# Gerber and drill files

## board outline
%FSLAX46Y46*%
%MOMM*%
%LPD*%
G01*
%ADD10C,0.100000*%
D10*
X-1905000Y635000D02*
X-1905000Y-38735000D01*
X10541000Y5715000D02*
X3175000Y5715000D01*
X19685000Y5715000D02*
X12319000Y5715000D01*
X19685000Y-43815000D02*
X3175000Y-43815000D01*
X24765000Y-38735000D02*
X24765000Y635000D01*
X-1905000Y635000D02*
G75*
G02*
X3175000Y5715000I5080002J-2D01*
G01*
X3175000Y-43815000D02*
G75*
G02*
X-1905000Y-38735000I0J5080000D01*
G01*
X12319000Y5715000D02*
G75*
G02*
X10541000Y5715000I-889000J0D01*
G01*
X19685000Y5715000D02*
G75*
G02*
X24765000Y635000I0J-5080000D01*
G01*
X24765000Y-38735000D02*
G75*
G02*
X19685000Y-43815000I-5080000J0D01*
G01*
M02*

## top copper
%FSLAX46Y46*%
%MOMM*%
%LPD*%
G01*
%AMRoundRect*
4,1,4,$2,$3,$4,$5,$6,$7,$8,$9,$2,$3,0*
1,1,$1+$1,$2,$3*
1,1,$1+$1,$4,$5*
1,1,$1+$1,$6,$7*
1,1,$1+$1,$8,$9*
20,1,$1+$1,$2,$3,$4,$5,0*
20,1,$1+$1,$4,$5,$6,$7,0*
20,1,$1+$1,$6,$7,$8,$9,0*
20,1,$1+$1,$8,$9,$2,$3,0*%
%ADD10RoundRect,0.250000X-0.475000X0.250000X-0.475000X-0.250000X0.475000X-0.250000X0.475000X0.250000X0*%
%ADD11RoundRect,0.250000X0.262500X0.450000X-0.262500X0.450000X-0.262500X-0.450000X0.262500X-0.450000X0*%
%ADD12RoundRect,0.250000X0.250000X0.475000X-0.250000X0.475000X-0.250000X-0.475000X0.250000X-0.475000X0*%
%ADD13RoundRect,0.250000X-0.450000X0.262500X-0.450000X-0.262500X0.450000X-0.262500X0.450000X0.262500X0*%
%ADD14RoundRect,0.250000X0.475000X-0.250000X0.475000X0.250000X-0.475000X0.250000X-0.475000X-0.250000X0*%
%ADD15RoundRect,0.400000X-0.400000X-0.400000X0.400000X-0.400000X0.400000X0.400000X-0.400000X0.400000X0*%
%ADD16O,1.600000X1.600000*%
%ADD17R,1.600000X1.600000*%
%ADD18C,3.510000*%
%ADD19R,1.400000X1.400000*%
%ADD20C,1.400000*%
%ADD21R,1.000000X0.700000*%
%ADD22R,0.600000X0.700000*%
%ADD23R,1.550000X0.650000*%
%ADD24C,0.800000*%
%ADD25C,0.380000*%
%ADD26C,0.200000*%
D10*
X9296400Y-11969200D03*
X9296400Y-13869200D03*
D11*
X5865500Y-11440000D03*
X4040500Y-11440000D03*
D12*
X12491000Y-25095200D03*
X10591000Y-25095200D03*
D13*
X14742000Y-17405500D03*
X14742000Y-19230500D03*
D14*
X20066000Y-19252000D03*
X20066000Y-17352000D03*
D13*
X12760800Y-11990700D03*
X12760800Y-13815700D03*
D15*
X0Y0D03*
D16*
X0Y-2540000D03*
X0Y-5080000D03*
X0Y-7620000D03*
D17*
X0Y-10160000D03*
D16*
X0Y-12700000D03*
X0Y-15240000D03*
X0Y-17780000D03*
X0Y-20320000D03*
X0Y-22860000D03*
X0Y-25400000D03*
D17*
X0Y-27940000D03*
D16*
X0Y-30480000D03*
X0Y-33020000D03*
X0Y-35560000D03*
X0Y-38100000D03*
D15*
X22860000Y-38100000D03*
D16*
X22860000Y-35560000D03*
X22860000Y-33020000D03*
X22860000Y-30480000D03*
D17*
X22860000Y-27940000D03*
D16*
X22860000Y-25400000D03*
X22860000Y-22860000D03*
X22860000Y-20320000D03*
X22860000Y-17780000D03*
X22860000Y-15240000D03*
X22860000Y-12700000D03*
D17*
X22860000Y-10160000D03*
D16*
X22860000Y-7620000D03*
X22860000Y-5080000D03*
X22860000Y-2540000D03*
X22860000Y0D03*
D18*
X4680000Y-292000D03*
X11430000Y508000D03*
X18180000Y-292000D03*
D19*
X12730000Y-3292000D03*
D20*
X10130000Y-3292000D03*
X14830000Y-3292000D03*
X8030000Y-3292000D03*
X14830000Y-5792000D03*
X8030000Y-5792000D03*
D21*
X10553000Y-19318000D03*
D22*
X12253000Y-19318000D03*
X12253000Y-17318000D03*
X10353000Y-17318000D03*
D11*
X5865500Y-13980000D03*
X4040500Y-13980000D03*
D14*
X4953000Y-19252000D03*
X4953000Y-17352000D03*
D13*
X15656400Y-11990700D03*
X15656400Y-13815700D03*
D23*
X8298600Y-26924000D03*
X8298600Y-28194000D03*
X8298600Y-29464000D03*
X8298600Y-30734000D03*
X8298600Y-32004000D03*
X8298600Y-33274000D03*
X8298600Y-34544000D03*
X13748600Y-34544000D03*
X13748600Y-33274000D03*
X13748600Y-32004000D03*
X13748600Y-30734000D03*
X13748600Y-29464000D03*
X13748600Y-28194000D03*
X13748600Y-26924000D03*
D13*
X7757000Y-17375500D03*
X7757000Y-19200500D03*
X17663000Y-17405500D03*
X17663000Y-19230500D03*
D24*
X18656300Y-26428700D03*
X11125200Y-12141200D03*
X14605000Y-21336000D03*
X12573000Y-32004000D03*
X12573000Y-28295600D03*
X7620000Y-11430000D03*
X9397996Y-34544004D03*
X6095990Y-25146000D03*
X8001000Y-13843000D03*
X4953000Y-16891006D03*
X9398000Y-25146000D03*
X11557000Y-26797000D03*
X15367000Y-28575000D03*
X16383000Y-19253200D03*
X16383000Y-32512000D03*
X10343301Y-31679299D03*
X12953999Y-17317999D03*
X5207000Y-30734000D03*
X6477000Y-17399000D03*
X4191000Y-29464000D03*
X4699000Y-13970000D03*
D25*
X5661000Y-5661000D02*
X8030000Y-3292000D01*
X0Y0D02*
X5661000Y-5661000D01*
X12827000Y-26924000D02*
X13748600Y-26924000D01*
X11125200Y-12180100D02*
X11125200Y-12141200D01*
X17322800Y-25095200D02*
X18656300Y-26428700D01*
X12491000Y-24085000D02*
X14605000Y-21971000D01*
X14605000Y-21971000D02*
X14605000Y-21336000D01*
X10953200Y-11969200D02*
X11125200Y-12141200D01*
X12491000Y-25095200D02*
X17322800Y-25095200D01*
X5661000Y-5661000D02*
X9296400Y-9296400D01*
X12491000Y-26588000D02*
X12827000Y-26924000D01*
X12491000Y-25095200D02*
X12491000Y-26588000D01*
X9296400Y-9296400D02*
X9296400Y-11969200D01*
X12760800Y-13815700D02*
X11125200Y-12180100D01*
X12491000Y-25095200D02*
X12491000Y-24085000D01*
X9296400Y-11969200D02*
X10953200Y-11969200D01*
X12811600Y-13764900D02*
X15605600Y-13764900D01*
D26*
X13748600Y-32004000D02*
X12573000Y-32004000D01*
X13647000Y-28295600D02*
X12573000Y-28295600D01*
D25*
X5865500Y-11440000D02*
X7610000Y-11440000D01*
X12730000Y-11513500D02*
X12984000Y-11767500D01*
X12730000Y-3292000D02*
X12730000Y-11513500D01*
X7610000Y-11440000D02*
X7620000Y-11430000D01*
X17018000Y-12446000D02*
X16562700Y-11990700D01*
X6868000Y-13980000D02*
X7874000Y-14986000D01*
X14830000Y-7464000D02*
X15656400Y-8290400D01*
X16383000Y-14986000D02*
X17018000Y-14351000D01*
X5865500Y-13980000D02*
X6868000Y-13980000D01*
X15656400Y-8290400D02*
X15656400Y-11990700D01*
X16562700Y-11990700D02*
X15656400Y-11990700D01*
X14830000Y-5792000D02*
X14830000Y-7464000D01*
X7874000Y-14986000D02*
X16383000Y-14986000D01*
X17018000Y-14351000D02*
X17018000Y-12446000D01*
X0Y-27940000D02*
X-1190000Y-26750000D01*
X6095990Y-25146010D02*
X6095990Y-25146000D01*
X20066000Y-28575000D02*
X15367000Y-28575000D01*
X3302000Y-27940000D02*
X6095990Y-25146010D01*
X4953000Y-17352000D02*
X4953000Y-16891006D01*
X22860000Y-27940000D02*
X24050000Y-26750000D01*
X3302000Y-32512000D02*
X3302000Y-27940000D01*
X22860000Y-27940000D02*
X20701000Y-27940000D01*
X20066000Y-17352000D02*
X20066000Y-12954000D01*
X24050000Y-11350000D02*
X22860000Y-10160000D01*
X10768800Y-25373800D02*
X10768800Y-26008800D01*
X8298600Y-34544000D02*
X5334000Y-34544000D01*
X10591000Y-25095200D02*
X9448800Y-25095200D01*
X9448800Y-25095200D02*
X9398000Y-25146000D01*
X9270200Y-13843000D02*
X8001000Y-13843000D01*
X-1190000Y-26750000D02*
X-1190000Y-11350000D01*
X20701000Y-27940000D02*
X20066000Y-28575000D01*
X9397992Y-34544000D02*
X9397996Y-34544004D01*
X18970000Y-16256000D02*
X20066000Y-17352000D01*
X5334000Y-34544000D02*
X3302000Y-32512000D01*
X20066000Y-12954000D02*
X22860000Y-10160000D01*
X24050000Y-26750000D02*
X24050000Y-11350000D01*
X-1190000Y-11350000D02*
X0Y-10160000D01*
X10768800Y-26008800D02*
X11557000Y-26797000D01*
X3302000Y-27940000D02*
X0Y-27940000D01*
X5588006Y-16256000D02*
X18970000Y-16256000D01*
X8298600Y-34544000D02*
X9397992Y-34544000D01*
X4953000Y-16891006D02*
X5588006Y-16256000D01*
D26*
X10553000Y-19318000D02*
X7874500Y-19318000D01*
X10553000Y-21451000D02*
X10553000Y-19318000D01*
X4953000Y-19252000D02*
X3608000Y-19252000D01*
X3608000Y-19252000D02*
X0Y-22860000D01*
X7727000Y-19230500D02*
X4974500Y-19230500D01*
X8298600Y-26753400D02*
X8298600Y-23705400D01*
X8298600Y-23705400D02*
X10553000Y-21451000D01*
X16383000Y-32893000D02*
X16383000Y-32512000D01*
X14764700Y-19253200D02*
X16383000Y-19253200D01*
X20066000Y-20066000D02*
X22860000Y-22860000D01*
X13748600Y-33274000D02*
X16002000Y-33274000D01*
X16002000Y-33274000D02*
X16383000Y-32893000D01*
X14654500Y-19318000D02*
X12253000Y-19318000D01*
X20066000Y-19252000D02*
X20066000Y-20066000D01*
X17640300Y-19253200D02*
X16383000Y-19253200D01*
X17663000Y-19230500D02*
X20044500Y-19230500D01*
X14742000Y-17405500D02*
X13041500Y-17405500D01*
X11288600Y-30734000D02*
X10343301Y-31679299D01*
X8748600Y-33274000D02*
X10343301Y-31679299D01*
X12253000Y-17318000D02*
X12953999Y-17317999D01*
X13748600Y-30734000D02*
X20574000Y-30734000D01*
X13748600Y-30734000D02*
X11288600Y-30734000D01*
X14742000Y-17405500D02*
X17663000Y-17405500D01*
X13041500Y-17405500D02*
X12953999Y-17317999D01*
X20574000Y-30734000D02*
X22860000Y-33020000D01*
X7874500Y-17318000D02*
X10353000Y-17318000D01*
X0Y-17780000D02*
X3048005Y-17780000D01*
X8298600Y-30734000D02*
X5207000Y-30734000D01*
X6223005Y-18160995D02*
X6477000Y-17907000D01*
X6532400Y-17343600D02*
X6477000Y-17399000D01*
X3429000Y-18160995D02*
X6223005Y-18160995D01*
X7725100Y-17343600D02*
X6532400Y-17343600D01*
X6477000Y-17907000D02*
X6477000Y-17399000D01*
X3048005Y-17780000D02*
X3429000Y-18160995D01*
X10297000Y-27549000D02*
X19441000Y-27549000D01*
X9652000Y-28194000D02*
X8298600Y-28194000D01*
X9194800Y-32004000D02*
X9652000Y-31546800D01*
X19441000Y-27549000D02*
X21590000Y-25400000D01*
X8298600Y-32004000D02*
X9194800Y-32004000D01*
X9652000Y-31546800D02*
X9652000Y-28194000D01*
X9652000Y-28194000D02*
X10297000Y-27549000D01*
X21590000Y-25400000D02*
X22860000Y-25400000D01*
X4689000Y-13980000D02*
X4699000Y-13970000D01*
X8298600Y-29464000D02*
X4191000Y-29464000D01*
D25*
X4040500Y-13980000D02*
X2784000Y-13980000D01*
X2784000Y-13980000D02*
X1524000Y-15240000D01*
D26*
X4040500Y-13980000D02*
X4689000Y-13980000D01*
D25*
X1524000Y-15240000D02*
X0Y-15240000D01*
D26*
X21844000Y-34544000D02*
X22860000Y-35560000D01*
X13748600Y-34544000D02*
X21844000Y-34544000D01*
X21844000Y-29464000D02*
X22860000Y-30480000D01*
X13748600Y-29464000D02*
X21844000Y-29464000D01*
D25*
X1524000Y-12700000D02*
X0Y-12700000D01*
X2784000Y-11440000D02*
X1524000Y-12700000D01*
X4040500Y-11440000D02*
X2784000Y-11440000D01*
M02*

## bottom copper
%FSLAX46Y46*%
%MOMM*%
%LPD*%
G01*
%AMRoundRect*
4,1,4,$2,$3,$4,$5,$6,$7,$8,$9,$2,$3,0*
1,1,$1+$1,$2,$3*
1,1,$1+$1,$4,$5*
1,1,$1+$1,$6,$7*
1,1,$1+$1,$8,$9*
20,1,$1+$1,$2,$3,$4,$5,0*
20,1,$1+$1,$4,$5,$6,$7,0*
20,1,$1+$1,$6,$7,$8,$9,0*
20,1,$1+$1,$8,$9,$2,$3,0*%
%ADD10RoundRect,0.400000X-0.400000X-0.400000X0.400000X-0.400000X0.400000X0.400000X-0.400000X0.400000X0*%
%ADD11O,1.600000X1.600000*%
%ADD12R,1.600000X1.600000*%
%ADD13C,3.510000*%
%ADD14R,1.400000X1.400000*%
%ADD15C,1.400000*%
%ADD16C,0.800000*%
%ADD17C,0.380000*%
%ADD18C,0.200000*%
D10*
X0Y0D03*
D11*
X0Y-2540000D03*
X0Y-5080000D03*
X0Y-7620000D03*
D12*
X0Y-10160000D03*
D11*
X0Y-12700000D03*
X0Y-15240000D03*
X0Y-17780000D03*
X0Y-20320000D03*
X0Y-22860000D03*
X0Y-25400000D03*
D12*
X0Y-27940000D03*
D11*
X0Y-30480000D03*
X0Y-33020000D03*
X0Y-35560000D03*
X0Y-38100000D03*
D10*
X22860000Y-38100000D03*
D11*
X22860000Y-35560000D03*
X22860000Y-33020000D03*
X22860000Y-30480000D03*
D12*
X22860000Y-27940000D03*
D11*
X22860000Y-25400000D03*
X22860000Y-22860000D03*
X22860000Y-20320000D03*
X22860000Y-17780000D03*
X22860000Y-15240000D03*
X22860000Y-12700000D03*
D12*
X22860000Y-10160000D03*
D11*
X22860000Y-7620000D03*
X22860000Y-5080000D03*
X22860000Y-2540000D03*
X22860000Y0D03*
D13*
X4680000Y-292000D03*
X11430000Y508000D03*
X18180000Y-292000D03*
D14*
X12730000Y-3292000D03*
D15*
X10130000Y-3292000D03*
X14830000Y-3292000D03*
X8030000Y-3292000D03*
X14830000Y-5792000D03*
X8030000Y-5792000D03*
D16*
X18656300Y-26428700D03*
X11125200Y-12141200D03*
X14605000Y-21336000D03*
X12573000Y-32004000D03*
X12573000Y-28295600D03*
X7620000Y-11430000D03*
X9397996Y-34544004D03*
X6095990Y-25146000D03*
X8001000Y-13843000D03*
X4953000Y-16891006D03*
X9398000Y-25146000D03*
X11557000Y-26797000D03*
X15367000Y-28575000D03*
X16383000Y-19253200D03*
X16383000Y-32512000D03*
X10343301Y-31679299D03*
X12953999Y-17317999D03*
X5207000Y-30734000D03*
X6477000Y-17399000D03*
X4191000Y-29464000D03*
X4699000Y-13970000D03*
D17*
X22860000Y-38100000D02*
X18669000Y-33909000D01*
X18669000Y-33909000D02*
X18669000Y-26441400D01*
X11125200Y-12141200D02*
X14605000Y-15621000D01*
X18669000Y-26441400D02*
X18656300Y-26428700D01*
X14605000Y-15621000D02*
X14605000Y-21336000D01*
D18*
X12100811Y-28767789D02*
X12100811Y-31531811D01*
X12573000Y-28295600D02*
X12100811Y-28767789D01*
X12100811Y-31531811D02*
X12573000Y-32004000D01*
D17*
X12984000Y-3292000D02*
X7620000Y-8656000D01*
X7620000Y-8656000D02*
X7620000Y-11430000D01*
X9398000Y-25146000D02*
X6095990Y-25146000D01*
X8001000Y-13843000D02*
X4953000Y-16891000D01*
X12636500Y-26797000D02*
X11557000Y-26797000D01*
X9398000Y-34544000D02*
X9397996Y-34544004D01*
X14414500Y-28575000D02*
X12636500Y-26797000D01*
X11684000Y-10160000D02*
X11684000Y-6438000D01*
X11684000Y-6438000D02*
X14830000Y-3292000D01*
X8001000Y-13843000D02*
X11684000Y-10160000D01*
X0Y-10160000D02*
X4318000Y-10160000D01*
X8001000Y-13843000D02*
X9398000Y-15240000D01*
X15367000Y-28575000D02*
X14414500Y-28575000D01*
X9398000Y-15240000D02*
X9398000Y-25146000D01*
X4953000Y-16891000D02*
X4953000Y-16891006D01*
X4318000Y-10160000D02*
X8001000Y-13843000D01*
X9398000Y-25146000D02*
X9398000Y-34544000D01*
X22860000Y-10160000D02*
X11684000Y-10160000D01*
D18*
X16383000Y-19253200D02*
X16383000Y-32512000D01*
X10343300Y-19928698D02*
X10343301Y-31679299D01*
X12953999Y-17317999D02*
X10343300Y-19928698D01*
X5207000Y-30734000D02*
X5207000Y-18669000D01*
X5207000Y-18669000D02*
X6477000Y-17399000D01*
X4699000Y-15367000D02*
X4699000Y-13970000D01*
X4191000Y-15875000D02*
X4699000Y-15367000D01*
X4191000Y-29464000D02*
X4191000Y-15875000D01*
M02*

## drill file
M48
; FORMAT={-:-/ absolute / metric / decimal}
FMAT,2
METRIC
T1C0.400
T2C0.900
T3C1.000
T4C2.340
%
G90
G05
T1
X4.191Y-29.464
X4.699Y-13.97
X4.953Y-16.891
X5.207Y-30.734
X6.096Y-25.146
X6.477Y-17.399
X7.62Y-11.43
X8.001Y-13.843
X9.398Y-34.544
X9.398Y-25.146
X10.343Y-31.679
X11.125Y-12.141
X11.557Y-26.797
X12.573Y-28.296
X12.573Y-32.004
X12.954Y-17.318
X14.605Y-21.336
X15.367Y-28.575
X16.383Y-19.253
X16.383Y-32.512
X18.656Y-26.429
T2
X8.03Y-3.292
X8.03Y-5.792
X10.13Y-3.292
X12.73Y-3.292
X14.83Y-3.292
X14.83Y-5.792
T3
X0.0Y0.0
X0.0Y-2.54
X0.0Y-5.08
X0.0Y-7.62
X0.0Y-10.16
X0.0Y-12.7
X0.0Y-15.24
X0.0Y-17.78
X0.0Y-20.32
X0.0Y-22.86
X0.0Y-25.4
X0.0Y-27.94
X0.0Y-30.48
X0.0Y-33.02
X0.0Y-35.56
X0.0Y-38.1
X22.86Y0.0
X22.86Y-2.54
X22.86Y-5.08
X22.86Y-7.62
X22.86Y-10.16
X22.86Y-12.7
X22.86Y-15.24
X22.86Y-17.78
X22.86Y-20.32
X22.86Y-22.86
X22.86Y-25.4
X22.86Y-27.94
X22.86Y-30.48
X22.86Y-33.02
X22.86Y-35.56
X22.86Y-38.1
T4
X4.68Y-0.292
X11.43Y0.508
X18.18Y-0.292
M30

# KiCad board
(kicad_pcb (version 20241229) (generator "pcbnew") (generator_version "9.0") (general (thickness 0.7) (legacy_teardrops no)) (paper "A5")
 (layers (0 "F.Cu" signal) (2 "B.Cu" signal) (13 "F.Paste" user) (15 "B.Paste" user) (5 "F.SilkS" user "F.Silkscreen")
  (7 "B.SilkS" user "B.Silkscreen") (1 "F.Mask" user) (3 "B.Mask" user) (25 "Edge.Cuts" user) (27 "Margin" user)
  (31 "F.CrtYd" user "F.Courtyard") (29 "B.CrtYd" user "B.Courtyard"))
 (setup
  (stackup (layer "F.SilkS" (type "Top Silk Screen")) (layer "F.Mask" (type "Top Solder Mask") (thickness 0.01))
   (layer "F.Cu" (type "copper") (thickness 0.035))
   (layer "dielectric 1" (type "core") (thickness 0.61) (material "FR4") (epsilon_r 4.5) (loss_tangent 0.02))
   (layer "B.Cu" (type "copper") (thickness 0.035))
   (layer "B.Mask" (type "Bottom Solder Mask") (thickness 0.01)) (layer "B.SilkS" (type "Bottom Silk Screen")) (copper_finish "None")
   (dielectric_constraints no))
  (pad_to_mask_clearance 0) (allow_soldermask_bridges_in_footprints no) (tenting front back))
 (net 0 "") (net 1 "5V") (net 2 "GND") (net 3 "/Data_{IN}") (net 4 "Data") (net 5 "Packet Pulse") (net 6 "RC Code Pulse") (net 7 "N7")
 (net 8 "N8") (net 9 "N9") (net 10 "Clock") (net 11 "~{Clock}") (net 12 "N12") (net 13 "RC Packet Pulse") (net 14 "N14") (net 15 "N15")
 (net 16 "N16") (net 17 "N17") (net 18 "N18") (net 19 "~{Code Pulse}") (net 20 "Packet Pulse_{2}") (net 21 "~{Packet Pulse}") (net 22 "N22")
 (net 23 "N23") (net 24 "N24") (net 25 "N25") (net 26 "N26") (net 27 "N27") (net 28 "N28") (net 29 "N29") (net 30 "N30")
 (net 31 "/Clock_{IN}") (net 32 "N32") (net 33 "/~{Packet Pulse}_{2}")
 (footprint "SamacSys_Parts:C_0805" (layer "F.Cu") (at 9.2964 12.9032 180)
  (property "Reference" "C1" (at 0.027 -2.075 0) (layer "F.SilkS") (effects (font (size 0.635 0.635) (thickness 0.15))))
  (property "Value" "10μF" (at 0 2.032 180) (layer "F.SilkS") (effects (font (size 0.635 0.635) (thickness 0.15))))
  (pad "1" smd roundrect (at 0 0.934 270) (size 1 1.45) (layers "F.Cu" "F.Mask" "F.Paste") (roundrect_rratio 0.25) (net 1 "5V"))
  (pad "2" smd roundrect (at 0 -0.966 270) (size 1 1.45) (layers "F.Cu" "F.Mask" "F.Paste") (roundrect_rratio 0.25) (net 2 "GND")))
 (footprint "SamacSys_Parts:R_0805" (layer "F.Cu") (at 4.953 11.43 90)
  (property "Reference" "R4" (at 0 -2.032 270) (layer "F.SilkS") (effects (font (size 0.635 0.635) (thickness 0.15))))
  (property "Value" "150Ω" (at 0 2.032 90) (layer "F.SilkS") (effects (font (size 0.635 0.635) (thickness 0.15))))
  (pad "1" smd roundrect (at -0.01 0.9125 180) (size 1.025 1.4) (layers "F.Cu" "F.Mask" "F.Paste") (roundrect_rratio 0.243902)
   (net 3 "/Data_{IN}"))
  (pad "2" smd roundrect (at -0.01 -0.9125 180) (size 1.025 1.4) (layers "F.Cu" "F.Mask" "F.Paste") (roundrect_rratio 0.243902)
   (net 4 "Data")))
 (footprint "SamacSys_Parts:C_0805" (layer "F.Cu") (at 11.557 25.0952 90)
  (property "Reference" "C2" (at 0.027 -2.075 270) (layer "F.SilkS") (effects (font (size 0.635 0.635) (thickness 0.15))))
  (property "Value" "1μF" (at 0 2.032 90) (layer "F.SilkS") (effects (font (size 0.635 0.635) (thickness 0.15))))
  (pad "1" smd roundrect (at 0 0.934 180) (size 1 1.45) (layers "F.Cu" "F.Mask" "F.Paste") (roundrect_rratio 0.25) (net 1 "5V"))
  (pad "2" smd roundrect (at 0 -0.966 180) (size 1 1.45) (layers "F.Cu" "F.Mask" "F.Paste") (roundrect_rratio 0.25) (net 2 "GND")))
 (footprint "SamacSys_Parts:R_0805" (layer "F.Cu") (at 14.732 18.318 180)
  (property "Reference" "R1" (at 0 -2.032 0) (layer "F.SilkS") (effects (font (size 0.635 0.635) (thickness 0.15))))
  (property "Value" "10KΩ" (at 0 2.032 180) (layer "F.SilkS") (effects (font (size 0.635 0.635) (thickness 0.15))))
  (pad "1" smd roundrect (at -0.01 0.9125 270) (size 1.025 1.4) (layers "F.Cu" "F.Mask" "F.Paste") (roundrect_rratio 0.243902)
   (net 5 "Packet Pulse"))
  (pad "2" smd roundrect (at -0.01 -0.9125 270) (size 1.025 1.4) (layers "F.Cu" "F.Mask" "F.Paste") (roundrect_rratio 0.243902)
   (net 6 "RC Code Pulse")))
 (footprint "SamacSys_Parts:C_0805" (layer "F.Cu") (at 20.066 18.318)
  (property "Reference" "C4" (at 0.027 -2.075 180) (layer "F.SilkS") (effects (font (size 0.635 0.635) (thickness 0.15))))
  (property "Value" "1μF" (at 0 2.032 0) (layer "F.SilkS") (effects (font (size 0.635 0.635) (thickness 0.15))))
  (pad "1" smd roundrect (at 0 0.934 90) (size 1 1.45) (layers "F.Cu" "F.Mask" "F.Paste") (roundrect_rratio 0.25) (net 6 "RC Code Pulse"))
  (pad "2" smd roundrect (at 0 -0.966 90) (size 1 1.45) (layers "F.Cu" "F.Mask" "F.Paste") (roundrect_rratio 0.25) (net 2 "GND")))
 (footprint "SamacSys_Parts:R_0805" (layer "F.Cu") (at 12.7508 12.9032 180)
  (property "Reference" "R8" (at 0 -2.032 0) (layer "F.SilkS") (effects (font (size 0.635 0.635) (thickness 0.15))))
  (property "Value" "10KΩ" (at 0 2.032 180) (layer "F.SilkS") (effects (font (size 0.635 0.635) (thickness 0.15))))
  (pad "1" smd roundrect (at -0.01 0.9125 270) (size 1.025 1.4) (layers "F.Cu" "F.Mask" "F.Paste") (roundrect_rratio 0.243902)
   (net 3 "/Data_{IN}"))
  (pad "2" smd roundrect (at -0.01 -0.9125 270) (size 1.025 1.4) (layers "F.Cu" "F.Mask" "F.Paste") (roundrect_rratio 0.243902) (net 1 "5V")))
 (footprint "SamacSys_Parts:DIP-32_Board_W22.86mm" (layer "F.Cu") (at 0 0)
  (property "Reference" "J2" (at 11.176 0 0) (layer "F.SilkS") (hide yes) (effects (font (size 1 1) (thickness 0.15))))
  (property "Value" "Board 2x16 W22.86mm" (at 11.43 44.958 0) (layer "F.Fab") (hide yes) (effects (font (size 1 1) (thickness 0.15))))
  (fp_line (start -1.905 -0.635) (end -1.905 38.735) (stroke (width 0.1) (type solid)) (layer "Edge.Cuts"))
  (fp_line (start 10.541 -5.715) (end 3.175 -5.715) (stroke (width 0.1) (type solid)) (layer "Edge.Cuts"))
  (fp_line (start 19.685 -5.715) (end 12.319 -5.715) (stroke (width 0.1) (type solid)) (layer "Edge.Cuts"))
  (fp_line (start 19.685 43.815) (end 3.175 43.815) (stroke (width 0.1) (type solid)) (layer "Edge.Cuts"))
  (fp_line (start 24.765 38.735) (end 24.765 -0.635) (stroke (width 0.1) (type solid)) (layer "Edge.Cuts"))
  (fp_arc (start -1.905 -0.635) (mid -0.417102 -4.227102) (end 3.175 -5.715) (stroke (width 0.1) (type solid)) (layer "Edge.Cuts"))
  (fp_arc (start 3.175 43.815) (mid -0.417102 42.327102) (end -1.905 38.735) (stroke (width 0.1) (type solid)) (layer "Edge.Cuts"))
  (fp_arc (start 12.319 -5.715) (mid 11.43 -4.826) (end 10.541 -5.715) (stroke (width 0.1) (type default)) (layer "Edge.Cuts"))
  (fp_arc (start 19.685 -5.715) (mid 23.277102 -4.227102) (end 24.765 -0.635) (stroke (width 0.1) (type solid)) (layer "Edge.Cuts"))
  (fp_arc (start 24.765 38.735) (mid 23.277103 42.327103) (end 19.685 43.815) (stroke (width 0.1) (type solid)) (layer "Edge.Cuts"))
  (pad "1" thru_hole roundrect (at 0 0) (size 1.6 1.6) (drill 1) (layers "*.Cu" "*.Mask") (remove_unused_layers no) (roundrect_rratio 0.25)
   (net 1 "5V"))
  (pad "2" thru_hole oval (at 0 2.54) (size 1.6 1.6) (drill 1) (layers "*.Cu" "*.Mask") (remove_unused_layers no) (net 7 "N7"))
  (pad "3" thru_hole oval (at 0 5.08) (size 1.6 1.6) (drill 1) (layers "*.Cu" "*.Mask") (remove_unused_layers no) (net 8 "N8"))
  (pad "4" thru_hole oval (at 0 7.62) (size 1.6 1.6) (drill 1) (layers "*.Cu" "*.Mask") (remove_unused_layers no) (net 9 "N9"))
  (pad "5" thru_hole rect (at 0 10.16) (size 1.6 1.6) (drill 1) (layers "*.Cu" "*.Mask") (remove_unused_layers no) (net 2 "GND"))
  (pad "6" thru_hole oval (at 0 12.7) (size 1.6 1.6) (drill 1) (layers "*.Cu" "*.Mask") (remove_unused_layers no) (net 4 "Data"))
  (pad "7" thru_hole oval (at 0 15.24) (size 1.6 1.6) (drill 1) (layers "*.Cu" "*.Mask") (remove_unused_layers no) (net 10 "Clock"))
  (pad "8" thru_hole oval (at 0 17.78) (size 1.6 1.6) (drill 1) (layers "*.Cu" "*.Mask") (remove_unused_layers no) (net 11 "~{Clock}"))
  (pad "9" thru_hole oval (at 0 20.32) (size 1.6 1.6) (drill 1) (layers "*.Cu" "*.Mask") (remove_unused_layers no) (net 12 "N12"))
  (pad "10" thru_hole oval (at 0 22.86) (size 1.6 1.6) (drill 1) (layers "*.Cu" "*.Mask") (remove_unused_layers no)
   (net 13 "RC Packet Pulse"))
  (pad "11" thru_hole oval (at 0 25.4) (size 1.6 1.6) (drill 1) (layers "*.Cu" "*.Mask") (remove_unused_layers no) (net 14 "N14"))
  (pad "12" thru_hole rect (at 0 27.94) (size 1.6 1.6) (drill 1) (layers "*.Cu" "*.Mask") (remove_unused_layers no) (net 2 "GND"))
  (pad "13" thru_hole oval (at 0 30.48) (size 1.6 1.6) (drill 1) (layers "*.Cu" "*.Mask") (remove_unused_layers no) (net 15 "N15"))
  (pad "14" thru_hole oval (at 0 33.02) (size 1.6 1.6) (drill 1) (layers "*.Cu" "*.Mask") (remove_unused_layers no) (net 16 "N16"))
  (pad "15" thru_hole oval (at 0 35.56) (size 1.6 1.6) (drill 1) (layers "*.Cu" "*.Mask") (remove_unused_layers no) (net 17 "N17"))
  (pad "16" thru_hole oval (at 0 38.1) (size 1.6 1.6) (drill 1) (layers "*.Cu" "*.Mask") (remove_unused_layers no) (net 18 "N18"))
  (pad "17" thru_hole roundrect (at 22.86 38.1) (size 1.6 1.6) (drill 1) (layers "*.Cu" "*.Mask") (remove_unused_layers no)
   (roundrect_rratio 0.25) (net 1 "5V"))
  (pad "18" thru_hole oval (at 22.86 35.56) (size 1.6 1.6) (drill 1) (layers "*.Cu" "*.Mask") (remove_unused_layers no)
   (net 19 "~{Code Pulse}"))
  (pad "19" thru_hole oval (at 22.86 33.02) (size 1.6 1.6) (drill 1) (layers "*.Cu" "*.Mask") (remove_unused_layers no)
   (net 5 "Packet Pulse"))
  (pad "20" thru_hole oval (at 22.86 30.48) (size 1.6 1.6) (drill 1) (layers "*.Cu" "*.Mask") (remove_unused_layers no)
   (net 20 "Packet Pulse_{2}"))
  (pad "21" thru_hole rect (at 22.86 27.94) (size 1.6 1.6) (drill 1) (layers "*.Cu" "*.Mask") (remove_unused_layers no) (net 2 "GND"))
  (pad "22" thru_hole oval (at 22.86 25.4) (size 1.6 1.6) (drill 1) (layers "*.Cu" "*.Mask") (remove_unused_layers no)
   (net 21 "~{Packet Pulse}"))
  (pad "23" thru_hole oval (at 22.86 22.86) (size 1.6 1.6) (drill 1) (layers "*.Cu" "*.Mask") (remove_unused_layers no)
   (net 6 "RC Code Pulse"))
  (pad "24" thru_hole oval (at 22.86 20.32) (size 1.6 1.6) (drill 1) (layers "*.Cu" "*.Mask") (remove_unused_layers no) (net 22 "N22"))
  (pad "25" thru_hole oval (at 22.86 17.78) (size 1.6 1.6) (drill 1) (layers "*.Cu" "*.Mask") (remove_unused_layers no) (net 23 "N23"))
  (pad "26" thru_hole oval (at 22.86 15.24) (size 1.6 1.6) (drill 1) (layers "*.Cu" "*.Mask") (remove_unused_layers no) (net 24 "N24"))
  (pad "27" thru_hole oval (at 22.86 12.7) (size 1.6 1.6) (drill 1) (layers "*.Cu" "*.Mask") (remove_unused_layers no) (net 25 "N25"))
  (pad "28" thru_hole rect (at 22.86 10.16) (size 1.6 1.6) (drill 1) (layers "*.Cu" "*.Mask") (remove_unused_layers no) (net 2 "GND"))
  (pad "29" thru_hole oval (at 22.86 7.62) (size 1.6 1.6) (drill 1) (layers "*.Cu" "*.Mask") (remove_unused_layers no) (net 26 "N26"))
  (pad "30" thru_hole oval (at 22.86 5.08) (size 1.6 1.6) (drill 1) (layers "*.Cu" "*.Mask") (remove_unused_layers no) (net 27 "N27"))
  (pad "31" thru_hole oval (at 22.86 2.54) (size 1.6 1.6) (drill 1) (layers "*.Cu" "*.Mask") (remove_unused_layers no) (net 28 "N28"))
  (pad "32" thru_hole oval (at 22.86 0) (size 1.6 1.6) (drill 1) (layers "*.Cu" "*.Mask") (remove_unused_layers no) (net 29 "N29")))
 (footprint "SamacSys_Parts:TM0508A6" (layer "F.Cu") (at 12.73 3.292)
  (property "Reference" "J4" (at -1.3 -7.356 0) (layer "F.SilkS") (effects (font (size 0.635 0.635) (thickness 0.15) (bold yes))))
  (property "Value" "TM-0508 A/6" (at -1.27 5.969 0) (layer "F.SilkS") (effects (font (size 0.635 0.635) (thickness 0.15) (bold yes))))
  (pad "" thru_hole circle (at -8.05 -3) (size 3.51 3.51) (drill 2.34) (layers "*.Cu" "*.Mask") (remove_unused_layers no))
  (pad "" thru_hole circle (at -1.3 -3.8) (size 3.51 3.51) (drill 2.34) (layers "*.Cu" "*.Mask") (remove_unused_layers no))
  (pad "" thru_hole circle (at 5.45 -3) (size 3.51 3.51) (drill 2.34) (layers "*.Cu" "*.Mask") (remove_unused_layers no))
  (pad "1" thru_hole rect (at 0 0) (size 1.4 1.4) (drill 0.9) (layers "*.Cu" "*.Mask") (remove_unused_layers no) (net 3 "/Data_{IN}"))
  (pad "2" thru_hole circle (at -2.6 0) (size 1.4 1.4) (drill 0.9) (layers "*.Cu" "*.Mask") (remove_unused_layers no) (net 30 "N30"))
  (pad "3" thru_hole circle (at 2.1 0) (size 1.4 1.4) (drill 0.9) (layers "*.Cu" "*.Mask") (remove_unused_layers no) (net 2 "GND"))
  (pad "4" thru_hole circle (at -4.7 0) (size 1.4 1.4) (drill 0.9) (layers "*.Cu" "*.Mask") (remove_unused_layers no) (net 1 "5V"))
  (pad "5" thru_hole circle (at 2.1 2.5) (size 1.4 1.4) (drill 0.9) (layers "*.Cu" "*.Mask") (remove_unused_layers no)
   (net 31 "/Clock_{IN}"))
  (pad "6" thru_hole circle (at -4.7 2.5) (size 1.4 1.4) (drill 0.9) (layers "*.Cu" "*.Mask") (remove_unused_layers no) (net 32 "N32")))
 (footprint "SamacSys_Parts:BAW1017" (layer "F.Cu") (at 11.303 18.318)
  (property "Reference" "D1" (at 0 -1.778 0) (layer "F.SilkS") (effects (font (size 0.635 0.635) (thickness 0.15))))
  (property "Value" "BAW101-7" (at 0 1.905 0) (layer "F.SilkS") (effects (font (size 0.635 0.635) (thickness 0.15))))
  (pad "1" smd rect (at -0.75 1 90) (size 0.7 1) (layers "F.Cu" "F.Mask" "F.Paste") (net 13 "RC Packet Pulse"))
  (pad "2" smd rect (at 0.95 1) (size 0.6 0.7) (layers "F.Cu" "F.Mask" "F.Paste") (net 6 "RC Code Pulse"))
  (pad "3" smd rect (at 0.95 -1) (size 0.6 0.7) (layers "F.Cu" "F.Mask" "F.Paste") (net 5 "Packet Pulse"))
  (pad "4" smd rect (at -0.95 -1) (size 0.6 0.7) (layers "F.Cu" "F.Mask" "F.Paste") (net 11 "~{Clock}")))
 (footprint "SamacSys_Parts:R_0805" (layer "F.Cu") (at 4.953 13.97 90)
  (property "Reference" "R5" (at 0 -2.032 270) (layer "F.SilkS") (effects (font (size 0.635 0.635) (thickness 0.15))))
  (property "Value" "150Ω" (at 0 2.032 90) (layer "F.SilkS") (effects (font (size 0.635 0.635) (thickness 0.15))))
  (pad "1" smd roundrect (at -0.01 0.9125 180) (size 1.025 1.4) (layers "F.Cu" "F.Mask" "F.Paste") (roundrect_rratio 0.243902)
   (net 31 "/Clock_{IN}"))
  (pad "2" smd roundrect (at -0.01 -0.9125 180) (size 1.025 1.4) (layers "F.Cu" "F.Mask" "F.Paste") (roundrect_rratio 0.243902)
   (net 10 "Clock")))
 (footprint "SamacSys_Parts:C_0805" (layer "F.Cu") (at 4.953 18.318)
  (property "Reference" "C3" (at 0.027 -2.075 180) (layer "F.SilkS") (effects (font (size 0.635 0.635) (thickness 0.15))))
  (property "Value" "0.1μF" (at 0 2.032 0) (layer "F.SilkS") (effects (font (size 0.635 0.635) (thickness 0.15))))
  (pad "1" smd roundrect (at 0 0.934 90) (size 1 1.45) (layers "F.Cu" "F.Mask" "F.Paste") (roundrect_rratio 0.25) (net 13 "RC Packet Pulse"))
  (pad "2" smd roundrect (at 0 -0.966 90) (size 1 1.45) (layers "F.Cu" "F.Mask" "F.Paste") (roundrect_rratio 0.25) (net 2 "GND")))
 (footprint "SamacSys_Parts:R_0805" (layer "F.Cu") (at 15.6464 12.9032 180)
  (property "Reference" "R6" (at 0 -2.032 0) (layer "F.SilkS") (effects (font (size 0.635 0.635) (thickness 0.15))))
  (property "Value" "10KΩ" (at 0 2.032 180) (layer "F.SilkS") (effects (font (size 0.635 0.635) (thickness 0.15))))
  (pad "1" smd roundrect (at -0.01 0.9125 270) (size 1.025 1.4) (layers "F.Cu" "F.Mask" "F.Paste") (roundrect_rratio 0.243902)
   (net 31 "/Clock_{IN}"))
  (pad "2" smd roundrect (at -0.01 -0.9125 270) (size 1.025 1.4) (layers "F.Cu" "F.Mask" "F.Paste") (roundrect_rratio 0.243902) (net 1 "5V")))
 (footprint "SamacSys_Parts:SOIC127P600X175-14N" (layer "F.Cu") (at 11.0236 30.734)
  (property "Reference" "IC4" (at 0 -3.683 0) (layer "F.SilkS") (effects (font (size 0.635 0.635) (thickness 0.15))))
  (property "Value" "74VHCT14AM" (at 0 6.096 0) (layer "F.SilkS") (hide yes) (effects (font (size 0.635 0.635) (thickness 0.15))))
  (pad "1" smd rect (at -2.725 -3.81 90) (size 0.65 1.55) (layers "F.Cu" "F.Mask" "F.Paste") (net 13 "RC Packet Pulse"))
  (pad "2" smd rect (at -2.725 -2.54 90) (size 0.65 1.55) (layers "F.Cu" "F.Mask" "F.Paste") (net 21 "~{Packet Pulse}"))
  (pad "3" smd rect (at -2.725 -1.27 90) (size 0.65 1.55) (layers "F.Cu" "F.Mask" "F.Paste") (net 10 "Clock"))
  (pad "4" smd rect (at -2.725 0 90) (size 0.65 1.55) (layers "F.Cu" "F.Mask" "F.Paste") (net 11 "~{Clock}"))
  (pad "5" smd rect (at -2.725 1.27 90) (size 0.65 1.55) (layers "F.Cu" "F.Mask" "F.Paste") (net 21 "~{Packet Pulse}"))
  (pad "6" smd rect (at -2.725 2.54 90) (size 0.65 1.55) (layers "F.Cu" "F.Mask" "F.Paste") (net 5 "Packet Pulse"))
  (pad "7" smd rect (at -2.725 3.81 90) (size 0.65 1.55) (layers "F.Cu" "F.Mask" "F.Paste") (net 2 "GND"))
  (pad "8" smd rect (at 2.725 3.81 90) (size 0.65 1.55) (layers "F.Cu" "F.Mask" "F.Paste") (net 19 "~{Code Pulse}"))
  (pad "9" smd rect (at 2.725 2.54 90) (size 0.65 1.55) (layers "F.Cu" "F.Mask" "F.Paste") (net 6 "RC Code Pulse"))
  (pad "10" smd rect (at 2.725 1.27 90) (size 0.65 1.55) (layers "F.Cu" "F.Mask" "F.Paste") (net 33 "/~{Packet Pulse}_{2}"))
  (pad "11" smd rect (at 2.725 0 90) (size 0.65 1.55) (layers "F.Cu" "F.Mask" "F.Paste") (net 5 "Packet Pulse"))
  (pad "12" smd rect (at 2.725 -1.27 90) (size 0.65 1.55) (layers "F.Cu" "F.Mask" "F.Paste") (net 20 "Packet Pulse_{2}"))
  (pad "13" smd rect (at 2.725 -2.54 90) (size 0.65 1.55) (layers "F.Cu" "F.Mask" "F.Paste") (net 33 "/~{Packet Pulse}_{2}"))
  (pad "14" smd rect (at 2.725 -3.81 90) (size 0.65 1.55) (layers "F.Cu" "F.Mask" "F.Paste") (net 1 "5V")))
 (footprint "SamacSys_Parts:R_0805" (layer "F.Cu") (at 7.747 18.288 180)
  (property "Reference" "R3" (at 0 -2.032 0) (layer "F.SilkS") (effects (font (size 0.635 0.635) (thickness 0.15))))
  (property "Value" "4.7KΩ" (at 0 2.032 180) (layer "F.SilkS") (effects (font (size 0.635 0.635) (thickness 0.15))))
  (pad "1" smd roundrect (at -0.01 0.9125 270) (size 1.025 1.4) (layers "F.Cu" "F.Mask" "F.Paste") (roundrect_rratio 0.243902)
   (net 11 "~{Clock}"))
  (pad "2" smd roundrect (at -0.01 -0.9125 270) (size 1.025 1.4) (layers "F.Cu" "F.Mask" "F.Paste") (roundrect_rratio 0.243902)
   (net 13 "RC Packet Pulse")))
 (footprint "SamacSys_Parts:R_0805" (layer "F.Cu") (at 17.653 18.318 180)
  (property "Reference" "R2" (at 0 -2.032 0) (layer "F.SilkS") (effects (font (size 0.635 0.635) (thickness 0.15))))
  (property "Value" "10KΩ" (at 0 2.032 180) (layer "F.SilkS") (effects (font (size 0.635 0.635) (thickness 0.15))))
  (pad "1" smd roundrect (at -0.01 0.9125 270) (size 1.025 1.4) (layers "F.Cu" "F.Mask" "F.Paste") (roundrect_rratio 0.243902)
   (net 5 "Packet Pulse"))
  (pad "2" smd roundrect (at -0.01 -0.9125 270) (size 1.025 1.4) (layers "F.Cu" "F.Mask" "F.Paste") (roundrect_rratio 0.243902)
   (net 6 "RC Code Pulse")))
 (segment (start 5.661 5.661) (end 8.03 3.292) (width 0.38) (layer "F.Cu") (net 1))
 (segment (start 0 0) (end 5.661 5.661) (width 0.38) (layer "F.Cu") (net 1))
 (segment (start 12.827 26.924) (end 13.7486 26.924) (width 0.38) (layer "F.Cu") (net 1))
 (segment (start 11.1252 12.1801) (end 11.1252 12.1412) (width 0.38) (layer "F.Cu") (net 1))
 (segment (start 17.3228 25.0952) (end 18.6563 26.4287) (width 0.38) (layer "F.Cu") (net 1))
 (segment (start 12.491 24.085) (end 14.605 21.971) (width 0.38) (layer "F.Cu") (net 1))
 (segment (start 14.605 21.971) (end 14.605 21.336) (width 0.38) (layer "F.Cu") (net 1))
 (segment (start 10.9532 11.9692) (end 11.1252 12.1412) (width 0.38) (layer "F.Cu") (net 1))
 (segment (start 12.491 25.0952) (end 17.3228 25.0952) (width 0.38) (layer "F.Cu") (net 1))
 (segment (start 5.661 5.661) (end 9.2964 9.2964) (width 0.38) (layer "F.Cu") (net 1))
 (segment (start 12.491 26.588) (end 12.827 26.924) (width 0.38) (layer "F.Cu") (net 1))
 (segment (start 12.491 25.0952) (end 12.491 26.588) (width 0.38) (layer "F.Cu") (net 1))
 (segment (start 9.2964 9.2964) (end 9.2964 11.9692) (width 0.38) (layer "F.Cu") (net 1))
 (segment (start 12.7608 13.8157) (end 11.1252 12.1801) (width 0.38) (layer "F.Cu") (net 1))
 (segment (start 12.491 25.0952) (end 12.491 24.085) (width 0.38) (layer "F.Cu") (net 1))
 (segment (start 9.2964 11.9692) (end 10.9532 11.9692) (width 0.38) (layer "F.Cu") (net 1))
 (segment (start 12.8116 13.7649) (end 15.6056 13.7649) (width 0.38) (layer "F.Cu") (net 1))
 (via (at 18.6563 26.4287) (size 0.8) (drill 0.4) (layers "F.Cu" "B.Cu") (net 1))
 (via (at 11.1252 12.1412) (size 0.8) (drill 0.4) (layers "F.Cu" "B.Cu") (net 1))
 (via (at 14.605 21.336) (size 0.8) (drill 0.4) (layers "F.Cu" "B.Cu") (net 1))
 (segment (start 22.86 38.1) (end 18.669 33.909) (width 0.38) (layer "B.Cu") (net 1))
 (segment (start 18.669 33.909) (end 18.669 26.4414) (width 0.38) (layer "B.Cu") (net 1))
 (segment (start 11.1252 12.1412) (end 14.605 15.621) (width 0.38) (layer "B.Cu") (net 1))
 (segment (start 18.669 26.4414) (end 18.6563 26.4287) (width 0.38) (layer "B.Cu") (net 1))
 (segment (start 14.605 15.621) (end 14.605 21.336) (width 0.38) (layer "B.Cu") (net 1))
 (segment (start 13.7486 32.004) (end 12.573 32.004) (width 0.2) (layer "F.Cu") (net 33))
 (segment (start 13.647 28.2956) (end 12.573 28.2956) (width 0.2) (layer "F.Cu") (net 33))
 (via (at 12.573 32.004) (size 0.8) (drill 0.4) (layers "F.Cu" "B.Cu") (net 33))
 (via (at 12.573 28.2956) (size 0.8) (drill 0.4) (layers "F.Cu" "B.Cu") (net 33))
 (segment (start 12.100811 28.767789) (end 12.100811 31.531811) (width 0.2) (layer "B.Cu") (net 33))
 (segment (start 12.573 28.2956) (end 12.100811 28.767789) (width 0.2) (layer "B.Cu") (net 33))
 (segment (start 12.100811 31.531811) (end 12.573 32.004) (width 0.2) (layer "B.Cu") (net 33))
 (segment (start 5.8655 11.44) (end 7.61 11.44) (width 0.38) (layer "F.Cu") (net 3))
 (segment (start 12.73 11.5135) (end 12.984 11.7675) (width 0.38) (layer "F.Cu") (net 3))
 (segment (start 12.73 3.292) (end 12.73 11.5135) (width 0.38) (layer "F.Cu") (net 3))
 (segment (start 7.61 11.44) (end 7.62 11.43) (width 0.38) (layer "F.Cu") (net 3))
 (via (at 7.62 11.43) (size 0.8) (drill 0.4) (layers "F.Cu" "B.Cu") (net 3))
 (segment (start 12.984 3.292) (end 7.62 8.656) (width 0.38) (layer "B.Cu") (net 3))
 (segment (start 7.62 8.656) (end 7.62 11.43) (width 0.38) (layer "B.Cu") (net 3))
 (segment (start 17.018 12.446) (end 16.5627 11.9907) (width 0.38) (layer "F.Cu") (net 31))
 (segment (start 6.868 13.98) (end 7.874 14.986) (width 0.38) (layer "F.Cu") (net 31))
 (segment (start 14.83 7.464) (end 15.6564 8.2904) (width 0.38) (layer "F.Cu") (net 31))
 (segment (start 16.383 14.986) (end 17.018 14.351) (width 0.38) (layer "F.Cu") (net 31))
 (segment (start 5.8655 13.98) (end 6.868 13.98) (width 0.38) (layer "F.Cu") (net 31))
 (segment (start 15.6564 8.2904) (end 15.6564 11.9907) (width 0.38) (layer "F.Cu") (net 31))
 (segment (start 16.5627 11.9907) (end 15.6564 11.9907) (width 0.38) (layer "F.Cu") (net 31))
 (segment (start 14.83 5.792) (end 14.83 7.464) (width 0.38) (layer "F.Cu") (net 31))
 (segment (start 7.874 14.986) (end 16.383 14.986) (width 0.38) (layer "F.Cu") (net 31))
 (segment (start 17.018 14.351) (end 17.018 12.446) (width 0.38) (layer "F.Cu") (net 31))
 (segment (start 0 27.94) (end -1.19 26.75) (width 0.38) (layer "F.Cu") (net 2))
 (segment (start 6.09599 25.14601) (end 6.09599 25.146) (width 0.38) (layer "F.Cu") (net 2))
 (segment (start 20.066 28.575) (end 15.367 28.575) (width 0.38) (layer "F.Cu") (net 2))
 (segment (start 3.302 27.94) (end 6.09599 25.14601) (width 0.38) (layer "F.Cu") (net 2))
 (segment (start 4.953 17.352) (end 4.953 16.891006) (width 0.38) (layer "F.Cu") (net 2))
 (segment (start 22.86 27.94) (end 24.05 26.75) (width 0.38) (layer "F.Cu") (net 2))
 (segment (start 3.302 32.512) (end 3.302 27.94) (width 0.38) (layer "F.Cu") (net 2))
 (segment (start 22.86 27.94) (end 20.701 27.94) (width 0.38) (layer "F.Cu") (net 2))
 (segment (start 20.066 17.352) (end 20.066 12.954) (width 0.38) (layer "F.Cu") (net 2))
 (segment (start 24.05 11.35) (end 22.86 10.16) (width 0.38) (layer "F.Cu") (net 2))
 (segment (start 10.7688 25.3738) (end 10.7688 26.0088) (width 0.38) (layer "F.Cu") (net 2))
 (segment (start 8.2986 34.544) (end 5.334 34.544) (width 0.38) (layer "F.Cu") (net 2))
 (segment (start 10.591 25.0952) (end 9.4488 25.0952) (width 0.38) (layer "F.Cu") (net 2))
 (segment (start 9.4488 25.0952) (end 9.398 25.146) (width 0.38) (layer "F.Cu") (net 2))
 (segment (start 9.2702 13.843) (end 8.001 13.843) (width 0.38) (layer "F.Cu") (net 2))
 (segment (start -1.19 26.75) (end -1.19 11.35) (width 0.38) (layer "F.Cu") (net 2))
 (segment (start 20.701 27.94) (end 20.066 28.575) (width 0.38) (layer "F.Cu") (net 2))
 (segment (start 9.397992 34.544) (end 9.397996 34.544004) (width 0.38) (layer "F.Cu") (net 2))
 (segment (start 18.97 16.256) (end 20.066 17.352) (width 0.38) (layer "F.Cu") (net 2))
 (segment (start 5.334 34.544) (end 3.302 32.512) (width 0.38) (layer "F.Cu") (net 2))
 (segment (start 20.066 12.954) (end 22.86 10.16) (width 0.38) (layer "F.Cu") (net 2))
 (segment (start 24.05 26.75) (end 24.05 11.35) (width 0.38) (layer "F.Cu") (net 2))
 (segment (start -1.19 11.35) (end 0 10.16) (width 0.38) (layer "F.Cu") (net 2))
 (segment (start 10.7688 26.0088) (end 11.557 26.797) (width 0.38) (layer "F.Cu") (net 2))
 (segment (start 3.302 27.94) (end 0 27.94) (width 0.38) (layer "F.Cu") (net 2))
 (segment (start 5.588006 16.256) (end 18.97 16.256) (width 0.38) (layer "F.Cu") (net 2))
 (segment (start 8.2986 34.544) (end 9.397992 34.544) (width 0.38) (layer "F.Cu") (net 2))
 (segment (start 4.953 16.891006) (end 5.588006 16.256) (width 0.38) (layer "F.Cu") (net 2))
 (via (at 9.397996 34.544004) (size 0.8) (drill 0.4) (layers "F.Cu" "B.Cu") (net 2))
 (via (at 6.09599 25.146) (size 0.8) (drill 0.4) (layers "F.Cu" "B.Cu") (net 2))
 (via (at 8.001 13.843) (size 0.8) (drill 0.4) (layers "F.Cu" "B.Cu") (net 2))
 (via (at 4.953 16.891006) (size 0.8) (drill 0.4) (layers "F.Cu" "B.Cu") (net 2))
 (via (at 9.398 25.146) (size 0.8) (drill 0.4) (layers "F.Cu" "B.Cu") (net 2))
 (via (at 11.557 26.797) (size 0.8) (drill 0.4) (layers "F.Cu" "B.Cu") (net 2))
 (via (at 15.367 28.575) (size 0.8) (drill 0.4) (layers "F.Cu" "B.Cu") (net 2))
 (segment (start 9.398 25.146) (end 6.09599 25.146) (width 0.38) (layer "B.Cu") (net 2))
 (segment (start 8.001 13.843) (end 4.953 16.891) (width 0.38) (layer "B.Cu") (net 2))
 (segment (start 12.6365 26.797) (end 11.557 26.797) (width 0.38) (layer "B.Cu") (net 2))
 (segment (start 9.398 34.544) (end 9.397996 34.544004) (width 0.38) (layer "B.Cu") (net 2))
 (segment (start 14.4145 28.575) (end 12.6365 26.797) (width 0.38) (layer "B.Cu") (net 2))
 (segment (start 11.684 10.16) (end 11.684 6.438) (width 0.38) (layer "B.Cu") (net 2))
 (segment (start 11.684 6.438) (end 14.83 3.292) (width 0.38) (layer "B.Cu") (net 2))
 (segment (start 8.001 13.843) (end 11.684 10.16) (width 0.38) (layer "B.Cu") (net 2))
 (segment (start 0 10.16) (end 4.318 10.16) (width 0.38) (layer "B.Cu") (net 2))
 (segment (start 8.001 13.843) (end 9.398 15.24) (width 0.38) (layer "B.Cu") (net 2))
 (segment (start 15.367 28.575) (end 14.4145 28.575) (width 0.38) (layer "B.Cu") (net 2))
 (segment (start 9.398 15.24) (end 9.398 25.146) (width 0.38) (layer "B.Cu") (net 2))
 (segment (start 4.953 16.891) (end 4.953 16.891006) (width 0.38) (layer "B.Cu") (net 2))
 (segment (start 4.318 10.16) (end 8.001 13.843) (width 0.38) (layer "B.Cu") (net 2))
 (segment (start 9.398 25.146) (end 9.398 34.544) (width 0.38) (layer "B.Cu") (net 2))
 (segment (start 22.86 10.16) (end 11.684 10.16) (width 0.38) (layer "B.Cu") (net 2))
 (segment (start 10.553 19.318) (end 7.8745 19.318) (width 0.2) (layer "F.Cu") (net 13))
 (segment (start 10.553 21.451) (end 10.553 19.318) (width 0.2) (layer "F.Cu") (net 13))
 (segment (start 4.953 19.252) (end 3.608 19.252) (width 0.2) (layer "F.Cu") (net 13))
 (segment (start 3.608 19.252) (end 0 22.86) (width 0.2) (layer "F.Cu") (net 13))
 (segment (start 7.727 19.2305) (end 4.9745 19.2305) (width 0.2) (layer "F.Cu") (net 13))
 (segment (start 8.2986 26.7534) (end 8.2986 23.7054) (width 0.2) (layer "F.Cu") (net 13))
 (segment (start 8.2986 23.7054) (end 10.553 21.451) (width 0.2) (layer "F.Cu") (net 13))
 (segment (start 16.383 32.893) (end 16.383 32.512) (width 0.2) (layer "F.Cu") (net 6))
 (segment (start 14.7647 19.2532) (end 16.383 19.2532) (width 0.2) (layer "F.Cu") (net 6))
 (segment (start 20.066 20.066) (end 22.86 22.86) (width 0.2) (layer "F.Cu") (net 6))
 (segment (start 13.7486 33.274) (end 16.002 33.274) (width 0.2) (layer "F.Cu") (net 6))
 (segment (start 16.002 33.274) (end 16.383 32.893) (width 0.2) (layer "F.Cu") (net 6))
 (segment (start 14.6545 19.318) (end 12.253 19.318) (width 0.2) (layer "F.Cu") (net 6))
 (segment (start 20.066 19.252) (end 20.066 20.066) (width 0.2) (layer "F.Cu") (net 6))
 (segment (start 17.6403 19.2532) (end 16.383 19.2532) (width 0.2) (layer "F.Cu") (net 6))
 (segment (start 17.663 19.2305) (end 20.0445 19.2305) (width 0.2) (layer "F.Cu") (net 6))
 (via (at 16.383 19.2532) (size 0.8) (drill 0.4) (layers "F.Cu" "B.Cu") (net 6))
 (via (at 16.383 32.512) (size 0.8) (drill 0.4) (layers "F.Cu" "B.Cu") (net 6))
 (segment (start 16.383 19.2532) (end 16.383 32.512) (width 0.2) (layer "B.Cu") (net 6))
 (segment (start 14.742 17.4055) (end 13.0415 17.4055) (width 0.2) (layer "F.Cu") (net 5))
 (segment (start 11.2886 30.734) (end 10.343301 31.679299) (width 0.2) (layer "F.Cu") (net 5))
 (segment (start 8.7486 33.274) (end 10.343301 31.679299) (width 0.2) (layer "F.Cu") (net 5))
 (segment (start 12.253 17.318) (end 12.953999 17.317999) (width 0.2) (layer "F.Cu") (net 5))
 (segment (start 13.7486 30.734) (end 20.574 30.734) (width 0.2) (layer "F.Cu") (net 5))
 (segment (start 13.7486 30.734) (end 11.2886 30.734) (width 0.2) (layer "F.Cu") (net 5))
 (segment (start 14.742 17.4055) (end 17.663 17.4055) (width 0.2) (layer "F.Cu") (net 5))
 (segment (start 13.0415 17.4055) (end 12.953999 17.317999) (width 0.2) (layer "F.Cu") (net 5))
 (segment (start 20.574 30.734) (end 22.86 33.02) (width 0.2) (layer "F.Cu") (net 5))
 (via (at 10.343301 31.679299) (size 0.8) (drill 0.4) (layers "F.Cu" "B.Cu") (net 5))
 (via (at 12.953999 17.317999) (size 0.8) (drill 0.4) (layers "F.Cu" "B.Cu") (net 5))
 (segment (start 10.3433 19.928698) (end 10.343301 31.679299) (width 0.2) (layer "B.Cu") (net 5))
 (segment (start 12.953999 17.317999) (end 10.3433 19.928698) (width 0.2) (layer "B.Cu") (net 5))
 (segment (start 7.8745 17.318) (end 10.353 17.318) (width 0.2) (layer "F.Cu") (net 11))
 (segment (start 0 17.78) (end 3.048005 17.78) (width 0.2) (layer "F.Cu") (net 11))
 (segment (start 8.2986 30.734) (end 5.207 30.734) (width 0.2) (layer "F.Cu") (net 11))
 (segment (start 6.223005 18.160995) (end 6.477 17.907) (width 0.2) (layer "F.Cu") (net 11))
 (segment (start 6.5324 17.3436) (end 6.477 17.399) (width 0.2) (layer "F.Cu") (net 11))
 (segment (start 3.429 18.160995) (end 6.223005 18.160995) (width 0.2) (layer "F.Cu") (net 11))
 (segment (start 7.7251 17.3436) (end 6.5324 17.3436) (width 0.2) (layer "F.Cu") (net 11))
 (segment (start 6.477 17.907) (end 6.477 17.399) (width 0.2) (layer "F.Cu") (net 11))
 (segment (start 3.048005 17.78) (end 3.429 18.160995) (width 0.2) (layer "F.Cu") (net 11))
 (via (at 5.207 30.734) (size 0.8) (drill 0.4) (layers "F.Cu" "B.Cu") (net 11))
 (via (at 6.477 17.399) (size 0.8) (drill 0.4) (layers "F.Cu" "B.Cu") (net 11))
 (segment (start 5.207 30.734) (end 5.207 18.669) (width 0.2) (layer "B.Cu") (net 11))
 (segment (start 5.207 18.669) (end 6.477 17.399) (width 0.2) (layer "B.Cu") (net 11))
 (segment (start 10.297 27.549) (end 19.441 27.549) (width 0.2) (layer "F.Cu") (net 21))
 (segment (start 9.652 28.194) (end 8.2986 28.194) (width 0.2) (layer "F.Cu") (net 21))
 (segment (start 9.1948 32.004) (end 9.652 31.5468) (width 0.2) (layer "F.Cu") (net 21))
 (segment (start 19.441 27.549) (end 21.59 25.4) (width 0.2) (layer "F.Cu") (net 21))
 (segment (start 8.2986 32.004) (end 9.1948 32.004) (width 0.2) (layer "F.Cu") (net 21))
 (segment (start 9.652 31.5468) (end 9.652 28.194) (width 0.2) (layer "F.Cu") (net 21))
 (segment (start 9.652 28.194) (end 10.297 27.549) (width 0.2) (layer "F.Cu") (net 21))
 (segment (start 21.59 25.4) (end 22.86 25.4) (width 0.2) (layer "F.Cu") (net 21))
 (segment (start 4.689 13.98) (end 4.699 13.97) (width 0.2) (layer "F.Cu") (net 10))
 (segment (start 8.2986 29.464) (end 4.191 29.464) (width 0.2) (layer "F.Cu") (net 10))
 (segment (start 4.0405 13.98) (end 2.784 13.98) (width 0.38) (layer "F.Cu") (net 10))
 (segment (start 2.784 13.98) (end 1.524 15.24) (width 0.38) (layer "F.Cu") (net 10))
 (segment (start 4.0405 13.98) (end 4.689 13.98) (width 0.2) (layer "F.Cu") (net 10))
 (segment (start 1.524 15.24) (end 0 15.24) (width 0.38) (layer "F.Cu") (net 10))
 (via (at 4.191 29.464) (size 0.8) (drill 0.4) (layers "F.Cu" "B.Cu") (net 10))
 (via (at 4.699 13.97) (size 0.8) (drill 0.4) (layers "F.Cu" "B.Cu") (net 10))
 (segment (start 4.699 15.367) (end 4.699 13.97) (width 0.2) (layer "B.Cu") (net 10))
 (segment (start 4.191 15.875) (end 4.699 15.367) (width 0.2) (layer "B.Cu") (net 10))
 (segment (start 4.191 29.464) (end 4.191 15.875) (width 0.2) (layer "B.Cu") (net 10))
 (segment (start 21.844 34.544) (end 22.86 35.56) (width 0.2) (layer "F.Cu") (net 19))
 (segment (start 13.7486 34.544) (end 21.844 34.544) (width 0.2) (layer "F.Cu") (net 19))
 (segment (start 21.844 29.464) (end 22.86 30.48) (width 0.2) (layer "F.Cu") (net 20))
 (segment (start 13.7486 29.464) (end 21.844 29.464) (width 0.2) (layer "F.Cu") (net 20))
 (segment (start 1.524 12.7) (end 0 12.7) (width 0.38) (layer "F.Cu") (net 4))
 (segment (start 2.784 11.44) (end 1.524 12.7) (width 0.38) (layer "F.Cu") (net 4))
 (segment (start 4.0405 11.44) (end 2.784 11.44) (width 0.38) (layer "F.Cu") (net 4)))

